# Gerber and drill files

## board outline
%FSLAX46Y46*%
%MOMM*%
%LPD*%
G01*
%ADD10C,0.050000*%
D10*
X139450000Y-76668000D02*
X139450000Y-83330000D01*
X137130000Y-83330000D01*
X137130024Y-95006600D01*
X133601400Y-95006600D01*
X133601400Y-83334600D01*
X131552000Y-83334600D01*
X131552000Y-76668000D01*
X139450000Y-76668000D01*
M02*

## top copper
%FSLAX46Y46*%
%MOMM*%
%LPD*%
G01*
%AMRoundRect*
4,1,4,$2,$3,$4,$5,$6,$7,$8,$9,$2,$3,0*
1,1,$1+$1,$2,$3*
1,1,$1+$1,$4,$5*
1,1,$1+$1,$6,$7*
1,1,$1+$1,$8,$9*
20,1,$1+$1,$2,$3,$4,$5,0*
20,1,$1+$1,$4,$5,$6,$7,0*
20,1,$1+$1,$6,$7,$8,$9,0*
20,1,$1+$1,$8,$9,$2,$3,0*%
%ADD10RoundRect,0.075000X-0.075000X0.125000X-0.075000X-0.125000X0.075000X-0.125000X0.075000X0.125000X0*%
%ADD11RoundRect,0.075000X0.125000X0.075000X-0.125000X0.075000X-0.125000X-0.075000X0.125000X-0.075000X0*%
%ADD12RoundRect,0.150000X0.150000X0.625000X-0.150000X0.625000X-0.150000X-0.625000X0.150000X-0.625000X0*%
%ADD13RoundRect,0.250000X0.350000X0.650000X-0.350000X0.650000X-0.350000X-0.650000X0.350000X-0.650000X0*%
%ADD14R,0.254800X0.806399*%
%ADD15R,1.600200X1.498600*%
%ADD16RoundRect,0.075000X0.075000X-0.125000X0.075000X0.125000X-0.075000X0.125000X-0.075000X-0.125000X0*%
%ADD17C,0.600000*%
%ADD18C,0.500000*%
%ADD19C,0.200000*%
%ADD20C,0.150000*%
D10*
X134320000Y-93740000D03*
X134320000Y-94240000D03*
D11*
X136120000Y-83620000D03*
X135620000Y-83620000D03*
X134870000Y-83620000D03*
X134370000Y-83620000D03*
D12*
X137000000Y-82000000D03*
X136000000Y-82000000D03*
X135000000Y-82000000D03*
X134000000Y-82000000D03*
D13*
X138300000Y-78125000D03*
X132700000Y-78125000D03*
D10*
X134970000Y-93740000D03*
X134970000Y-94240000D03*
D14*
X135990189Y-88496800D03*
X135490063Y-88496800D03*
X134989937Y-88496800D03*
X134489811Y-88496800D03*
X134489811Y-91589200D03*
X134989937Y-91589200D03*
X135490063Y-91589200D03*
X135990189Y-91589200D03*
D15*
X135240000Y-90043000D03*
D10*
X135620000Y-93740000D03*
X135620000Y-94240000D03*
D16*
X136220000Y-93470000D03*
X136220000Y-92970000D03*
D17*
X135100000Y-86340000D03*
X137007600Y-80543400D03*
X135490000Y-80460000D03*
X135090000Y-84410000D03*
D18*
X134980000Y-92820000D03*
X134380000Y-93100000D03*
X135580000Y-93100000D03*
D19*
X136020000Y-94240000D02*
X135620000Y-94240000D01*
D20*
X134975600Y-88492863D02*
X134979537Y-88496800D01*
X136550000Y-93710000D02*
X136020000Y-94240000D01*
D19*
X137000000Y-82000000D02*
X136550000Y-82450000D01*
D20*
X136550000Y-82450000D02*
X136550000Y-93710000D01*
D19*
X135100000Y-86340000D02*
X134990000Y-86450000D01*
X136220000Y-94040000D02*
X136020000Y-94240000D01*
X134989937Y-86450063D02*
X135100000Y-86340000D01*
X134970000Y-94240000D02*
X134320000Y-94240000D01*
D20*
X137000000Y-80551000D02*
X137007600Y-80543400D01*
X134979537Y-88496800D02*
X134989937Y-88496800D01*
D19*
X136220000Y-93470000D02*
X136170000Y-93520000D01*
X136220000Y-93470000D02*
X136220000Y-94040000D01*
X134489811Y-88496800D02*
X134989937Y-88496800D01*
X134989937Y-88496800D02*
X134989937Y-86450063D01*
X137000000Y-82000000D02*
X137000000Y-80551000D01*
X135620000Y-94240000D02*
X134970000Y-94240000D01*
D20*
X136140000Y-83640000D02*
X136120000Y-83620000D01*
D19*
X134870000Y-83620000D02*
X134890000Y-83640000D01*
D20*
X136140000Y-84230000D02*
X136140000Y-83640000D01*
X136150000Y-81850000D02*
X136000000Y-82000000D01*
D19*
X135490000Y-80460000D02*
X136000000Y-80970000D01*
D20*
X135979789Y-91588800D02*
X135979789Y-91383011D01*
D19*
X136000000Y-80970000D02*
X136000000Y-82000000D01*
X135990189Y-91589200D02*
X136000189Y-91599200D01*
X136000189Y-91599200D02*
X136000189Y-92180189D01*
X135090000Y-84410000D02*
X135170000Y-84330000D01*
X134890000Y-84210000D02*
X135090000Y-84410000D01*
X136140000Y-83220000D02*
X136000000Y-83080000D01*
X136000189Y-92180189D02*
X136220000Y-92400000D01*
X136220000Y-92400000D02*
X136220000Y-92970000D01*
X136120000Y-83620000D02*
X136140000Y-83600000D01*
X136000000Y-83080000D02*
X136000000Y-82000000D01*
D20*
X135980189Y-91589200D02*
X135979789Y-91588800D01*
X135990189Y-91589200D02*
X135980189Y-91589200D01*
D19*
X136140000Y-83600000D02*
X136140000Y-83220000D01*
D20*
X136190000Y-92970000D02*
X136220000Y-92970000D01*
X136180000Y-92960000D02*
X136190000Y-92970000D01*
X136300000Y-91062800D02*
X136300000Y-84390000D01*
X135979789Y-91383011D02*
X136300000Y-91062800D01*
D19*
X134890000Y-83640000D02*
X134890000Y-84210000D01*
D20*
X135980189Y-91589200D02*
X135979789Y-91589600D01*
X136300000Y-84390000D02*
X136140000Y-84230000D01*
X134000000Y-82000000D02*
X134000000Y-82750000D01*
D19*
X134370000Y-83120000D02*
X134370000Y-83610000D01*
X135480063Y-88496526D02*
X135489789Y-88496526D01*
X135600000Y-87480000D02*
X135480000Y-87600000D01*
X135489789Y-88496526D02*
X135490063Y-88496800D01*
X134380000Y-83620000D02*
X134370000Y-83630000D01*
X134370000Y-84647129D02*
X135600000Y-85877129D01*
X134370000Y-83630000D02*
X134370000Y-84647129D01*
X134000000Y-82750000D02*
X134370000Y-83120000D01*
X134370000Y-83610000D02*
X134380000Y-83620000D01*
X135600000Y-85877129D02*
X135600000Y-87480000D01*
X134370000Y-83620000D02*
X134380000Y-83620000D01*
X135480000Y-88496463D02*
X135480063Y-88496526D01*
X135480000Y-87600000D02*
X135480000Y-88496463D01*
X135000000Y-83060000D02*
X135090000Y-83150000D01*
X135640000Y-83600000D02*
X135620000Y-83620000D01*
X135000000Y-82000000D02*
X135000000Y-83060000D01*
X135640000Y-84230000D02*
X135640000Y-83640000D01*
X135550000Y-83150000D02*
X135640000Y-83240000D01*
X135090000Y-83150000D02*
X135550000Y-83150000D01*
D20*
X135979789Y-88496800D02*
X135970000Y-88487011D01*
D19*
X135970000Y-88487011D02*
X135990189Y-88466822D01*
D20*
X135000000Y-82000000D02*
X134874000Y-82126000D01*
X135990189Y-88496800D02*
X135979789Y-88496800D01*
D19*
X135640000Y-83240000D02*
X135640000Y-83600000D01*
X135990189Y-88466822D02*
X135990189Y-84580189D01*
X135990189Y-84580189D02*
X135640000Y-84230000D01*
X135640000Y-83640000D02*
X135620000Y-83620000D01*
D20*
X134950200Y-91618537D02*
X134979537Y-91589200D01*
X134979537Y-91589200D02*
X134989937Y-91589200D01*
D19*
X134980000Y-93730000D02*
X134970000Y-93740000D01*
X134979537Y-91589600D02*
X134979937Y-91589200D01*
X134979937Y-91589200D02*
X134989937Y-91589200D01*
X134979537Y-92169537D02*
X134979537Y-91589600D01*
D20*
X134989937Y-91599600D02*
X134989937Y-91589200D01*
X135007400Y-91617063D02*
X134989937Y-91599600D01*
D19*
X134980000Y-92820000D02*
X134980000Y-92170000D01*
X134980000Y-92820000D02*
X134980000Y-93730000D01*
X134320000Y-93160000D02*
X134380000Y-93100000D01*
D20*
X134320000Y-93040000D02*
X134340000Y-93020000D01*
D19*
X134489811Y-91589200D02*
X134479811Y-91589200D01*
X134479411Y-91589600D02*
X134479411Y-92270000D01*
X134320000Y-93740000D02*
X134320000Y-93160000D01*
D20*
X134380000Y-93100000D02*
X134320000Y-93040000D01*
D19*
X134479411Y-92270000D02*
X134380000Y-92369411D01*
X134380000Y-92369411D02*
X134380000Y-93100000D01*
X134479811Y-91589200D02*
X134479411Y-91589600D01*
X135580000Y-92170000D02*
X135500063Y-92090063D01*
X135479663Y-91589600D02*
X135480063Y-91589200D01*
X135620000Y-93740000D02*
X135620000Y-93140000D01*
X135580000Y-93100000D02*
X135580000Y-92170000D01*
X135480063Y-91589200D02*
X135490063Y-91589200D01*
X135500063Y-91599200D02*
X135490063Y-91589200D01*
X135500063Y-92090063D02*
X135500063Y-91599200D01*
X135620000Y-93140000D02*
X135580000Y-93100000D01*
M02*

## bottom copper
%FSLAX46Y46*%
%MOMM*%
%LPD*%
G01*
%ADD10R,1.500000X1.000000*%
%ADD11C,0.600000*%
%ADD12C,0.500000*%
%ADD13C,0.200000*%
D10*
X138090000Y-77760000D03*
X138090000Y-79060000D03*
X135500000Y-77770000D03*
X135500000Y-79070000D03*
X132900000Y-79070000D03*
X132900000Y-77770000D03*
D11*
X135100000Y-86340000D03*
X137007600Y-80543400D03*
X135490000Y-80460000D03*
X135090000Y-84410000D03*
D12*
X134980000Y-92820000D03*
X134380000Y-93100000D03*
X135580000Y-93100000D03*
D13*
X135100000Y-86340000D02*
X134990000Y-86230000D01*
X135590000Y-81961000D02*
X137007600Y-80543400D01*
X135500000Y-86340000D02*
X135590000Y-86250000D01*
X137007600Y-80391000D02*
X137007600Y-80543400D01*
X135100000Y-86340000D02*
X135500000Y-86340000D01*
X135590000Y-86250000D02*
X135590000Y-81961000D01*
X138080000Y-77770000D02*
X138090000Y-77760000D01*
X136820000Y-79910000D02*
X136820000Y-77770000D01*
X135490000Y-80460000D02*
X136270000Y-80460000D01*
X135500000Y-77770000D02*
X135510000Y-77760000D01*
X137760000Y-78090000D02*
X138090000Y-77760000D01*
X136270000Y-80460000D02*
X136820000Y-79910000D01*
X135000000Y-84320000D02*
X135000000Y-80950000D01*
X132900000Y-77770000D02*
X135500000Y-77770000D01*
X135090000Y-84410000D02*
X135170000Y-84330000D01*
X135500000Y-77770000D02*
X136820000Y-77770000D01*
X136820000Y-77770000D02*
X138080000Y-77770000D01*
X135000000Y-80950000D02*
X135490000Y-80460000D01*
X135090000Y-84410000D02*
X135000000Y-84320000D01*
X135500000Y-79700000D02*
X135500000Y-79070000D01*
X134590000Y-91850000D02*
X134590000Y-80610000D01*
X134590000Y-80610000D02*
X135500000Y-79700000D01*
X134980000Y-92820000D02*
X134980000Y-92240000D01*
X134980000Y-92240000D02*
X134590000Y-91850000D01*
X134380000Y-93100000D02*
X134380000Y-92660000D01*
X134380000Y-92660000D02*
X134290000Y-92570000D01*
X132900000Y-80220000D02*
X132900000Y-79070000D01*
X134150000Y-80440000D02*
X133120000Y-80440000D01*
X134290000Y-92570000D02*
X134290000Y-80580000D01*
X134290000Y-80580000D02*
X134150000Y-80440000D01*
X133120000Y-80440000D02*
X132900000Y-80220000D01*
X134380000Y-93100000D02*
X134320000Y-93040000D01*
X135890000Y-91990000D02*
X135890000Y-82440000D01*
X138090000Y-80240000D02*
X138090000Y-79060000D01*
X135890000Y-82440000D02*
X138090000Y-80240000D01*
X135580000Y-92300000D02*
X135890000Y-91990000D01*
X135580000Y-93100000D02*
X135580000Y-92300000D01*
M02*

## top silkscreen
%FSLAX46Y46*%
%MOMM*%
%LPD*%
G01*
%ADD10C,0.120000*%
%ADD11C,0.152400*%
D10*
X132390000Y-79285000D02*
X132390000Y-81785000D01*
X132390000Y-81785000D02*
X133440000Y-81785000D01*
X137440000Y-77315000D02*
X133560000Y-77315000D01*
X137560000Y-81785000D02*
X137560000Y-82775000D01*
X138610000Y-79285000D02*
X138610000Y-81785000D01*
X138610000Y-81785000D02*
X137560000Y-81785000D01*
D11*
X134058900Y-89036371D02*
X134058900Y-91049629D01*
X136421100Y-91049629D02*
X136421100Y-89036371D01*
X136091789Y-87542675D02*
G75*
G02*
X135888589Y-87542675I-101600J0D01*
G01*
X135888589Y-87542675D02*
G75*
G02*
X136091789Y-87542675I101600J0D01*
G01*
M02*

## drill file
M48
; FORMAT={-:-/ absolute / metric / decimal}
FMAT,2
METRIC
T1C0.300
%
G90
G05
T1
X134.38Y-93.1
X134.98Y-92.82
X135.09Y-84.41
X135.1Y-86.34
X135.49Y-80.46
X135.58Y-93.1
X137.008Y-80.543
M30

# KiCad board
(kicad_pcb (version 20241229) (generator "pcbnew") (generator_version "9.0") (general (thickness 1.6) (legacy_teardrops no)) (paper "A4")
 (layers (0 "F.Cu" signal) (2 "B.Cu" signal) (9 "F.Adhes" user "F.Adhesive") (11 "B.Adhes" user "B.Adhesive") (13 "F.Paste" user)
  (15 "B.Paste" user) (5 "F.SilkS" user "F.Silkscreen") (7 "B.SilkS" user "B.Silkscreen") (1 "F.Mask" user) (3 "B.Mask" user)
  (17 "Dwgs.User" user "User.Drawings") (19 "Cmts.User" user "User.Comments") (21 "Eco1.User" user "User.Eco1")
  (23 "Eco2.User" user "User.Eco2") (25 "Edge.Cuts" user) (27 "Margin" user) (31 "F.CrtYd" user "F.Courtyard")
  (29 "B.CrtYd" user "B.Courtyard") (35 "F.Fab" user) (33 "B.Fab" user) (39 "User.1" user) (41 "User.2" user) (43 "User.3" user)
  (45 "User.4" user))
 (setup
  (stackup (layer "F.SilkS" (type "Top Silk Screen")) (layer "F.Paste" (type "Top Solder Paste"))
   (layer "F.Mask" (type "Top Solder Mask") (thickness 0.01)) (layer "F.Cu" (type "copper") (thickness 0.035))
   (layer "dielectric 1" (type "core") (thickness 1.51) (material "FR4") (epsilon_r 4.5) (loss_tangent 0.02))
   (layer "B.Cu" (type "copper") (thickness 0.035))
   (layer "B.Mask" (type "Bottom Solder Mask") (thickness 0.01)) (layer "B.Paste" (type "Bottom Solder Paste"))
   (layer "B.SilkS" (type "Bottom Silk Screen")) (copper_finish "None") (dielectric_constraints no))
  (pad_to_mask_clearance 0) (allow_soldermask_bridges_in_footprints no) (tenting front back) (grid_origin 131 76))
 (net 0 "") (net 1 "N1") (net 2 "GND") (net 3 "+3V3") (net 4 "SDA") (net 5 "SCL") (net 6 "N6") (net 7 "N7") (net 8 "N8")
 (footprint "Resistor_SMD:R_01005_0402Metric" (layer "F.Cu") (at 134.32 93.99 -90)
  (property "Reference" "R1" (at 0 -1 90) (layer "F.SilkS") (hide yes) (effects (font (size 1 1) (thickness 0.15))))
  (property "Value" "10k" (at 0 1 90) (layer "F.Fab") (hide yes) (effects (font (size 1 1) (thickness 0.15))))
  (pad "" smd roundrect (at -0.275 0 270) (size 0.27 0.27) (layers "F.Paste") (roundrect_rratio 0.25))
  (pad "" smd roundrect (at 0.275 0 270) (size 0.27 0.27) (layers "F.Paste") (roundrect_rratio 0.25))
  (pad "1" smd roundrect (at -0.25 0 270) (size 0.4 0.3) (layers "F.Cu" "F.Mask") (roundrect_rratio 0.25) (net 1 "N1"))
  (pad "2" smd roundrect (at 0.25 0 270) (size 0.4 0.3) (layers "F.Cu" "F.Mask") (roundrect_rratio 0.25) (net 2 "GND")))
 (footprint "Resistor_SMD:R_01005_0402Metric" (layer "F.Cu") (at 135.87 83.62 180)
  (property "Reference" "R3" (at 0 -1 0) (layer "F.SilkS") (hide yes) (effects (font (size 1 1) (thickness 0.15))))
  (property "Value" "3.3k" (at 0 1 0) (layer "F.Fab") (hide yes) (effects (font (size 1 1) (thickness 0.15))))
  (pad "" smd roundrect (at -0.275 0 180) (size 0.27 0.27) (layers "F.Paste") (roundrect_rratio 0.25))
  (pad "" smd roundrect (at 0.275 0 180) (size 0.27 0.27) (layers "F.Paste") (roundrect_rratio 0.25))
  (pad "1" smd roundrect (at -0.25 0 180) (size 0.4 0.3) (layers "F.Cu" "F.Mask") (roundrect_rratio 0.25) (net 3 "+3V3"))
  (pad "2" smd roundrect (at 0.25 0 180) (size 0.4 0.3) (layers "F.Cu" "F.Mask") (roundrect_rratio 0.25) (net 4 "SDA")))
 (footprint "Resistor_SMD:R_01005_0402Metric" (layer "F.Cu") (at 134.62 83.62 180)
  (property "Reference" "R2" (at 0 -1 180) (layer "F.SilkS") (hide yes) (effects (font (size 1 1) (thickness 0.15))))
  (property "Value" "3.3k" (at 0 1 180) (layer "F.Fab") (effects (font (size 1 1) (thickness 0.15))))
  (pad "" smd roundrect (at -0.275 0 180) (size 0.27 0.27) (layers "F.Paste") (roundrect_rratio 0.25))
  (pad "" smd roundrect (at 0.275 0 180) (size 0.27 0.27) (layers "F.Paste") (roundrect_rratio 0.25))
  (pad "1" smd roundrect (at -0.25 0 180) (size 0.4 0.3) (layers "F.Cu" "F.Mask") (roundrect_rratio 0.25) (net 3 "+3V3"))
  (pad "2" smd roundrect (at 0.25 0 180) (size 0.4 0.3) (layers "F.Cu" "F.Mask") (roundrect_rratio 0.25) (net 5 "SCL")))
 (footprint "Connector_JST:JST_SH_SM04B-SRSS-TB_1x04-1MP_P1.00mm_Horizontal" (layer "F.Cu") (at 135.5 80 180)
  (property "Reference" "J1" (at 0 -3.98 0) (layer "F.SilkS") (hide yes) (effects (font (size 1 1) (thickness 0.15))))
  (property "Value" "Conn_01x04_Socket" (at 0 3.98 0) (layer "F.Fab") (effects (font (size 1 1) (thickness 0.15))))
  (fp_line (start 3.11 0.715) (end 3.11 -1.785) (stroke (width 0.12) (type solid)) (layer "F.SilkS"))
  (fp_line (start 3.11 -1.785) (end 2.06 -1.785) (stroke (width 0.12) (type solid)) (layer "F.SilkS"))
  (fp_line (start -1.94 2.685) (end 1.94 2.685) (stroke (width 0.12) (type solid)) (layer "F.SilkS"))
  (fp_line (start -2.06 -1.785) (end -2.06 -2.775) (stroke (width 0.12) (type solid)) (layer "F.SilkS"))
  (fp_line (start -3.11 0.715) (end -3.11 -1.785) (stroke (width 0.12) (type solid)) (layer "F.SilkS"))
  (fp_line (start -3.11 -1.785) (end -2.06 -1.785) (stroke (width 0.12) (type solid)) (layer "F.SilkS"))
  (pad "1" smd roundrect (at -1.5 -2 180) (size 0.6 1.55) (layers "F.Cu" "F.Mask" "F.Paste") (roundrect_rratio 0.25) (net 2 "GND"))
  (pad "2" smd roundrect (at -0.5 -2 180) (size 0.6 1.55) (layers "F.Cu" "F.Mask" "F.Paste") (roundrect_rratio 0.25) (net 3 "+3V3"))
  (pad "3" smd roundrect (at 0.5 -2 180) (size 0.6 1.55) (layers "F.Cu" "F.Mask" "F.Paste") (roundrect_rratio 0.25) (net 4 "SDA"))
  (pad "4" smd roundrect (at 1.5 -2 180) (size 0.6 1.55) (layers "F.Cu" "F.Mask" "F.Paste") (roundrect_rratio 0.25) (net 5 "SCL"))
  (pad "MP" smd roundrect (at -2.8 1.875 180) (size 1.2 1.8) (layers "F.Cu" "F.Mask" "F.Paste") (roundrect_rratio 0.208333))
  (pad "MP" smd roundrect (at 2.8 1.875 180) (size 1.2 1.8) (layers "F.Cu" "F.Mask" "F.Paste") (roundrect_rratio 0.208333)))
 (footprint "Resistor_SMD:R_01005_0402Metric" (layer "F.Cu") (at 134.97 93.99 -90)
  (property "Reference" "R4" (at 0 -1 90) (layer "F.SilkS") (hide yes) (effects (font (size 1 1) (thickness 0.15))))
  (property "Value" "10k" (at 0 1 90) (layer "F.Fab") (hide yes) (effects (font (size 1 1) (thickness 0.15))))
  (pad "" smd roundrect (at -0.275 0 270) (size 0.27 0.27) (layers "F.Paste") (roundrect_rratio 0.25))
  (pad "" smd roundrect (at 0.275 0 270) (size 0.27 0.27) (layers "F.Paste") (roundrect_rratio 0.25))
  (pad "1" smd roundrect (at -0.25 0 270) (size 0.4 0.3) (layers "F.Cu" "F.Mask") (roundrect_rratio 0.25) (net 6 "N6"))
  (pad "2" smd roundrect (at 0.25 0 270) (size 0.4 0.3) (layers "F.Cu" "F.Mask") (roundrect_rratio 0.25) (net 2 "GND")))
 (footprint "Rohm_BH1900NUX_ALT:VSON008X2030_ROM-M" (layer "F.Cu") (at 135.24 90.043 -90)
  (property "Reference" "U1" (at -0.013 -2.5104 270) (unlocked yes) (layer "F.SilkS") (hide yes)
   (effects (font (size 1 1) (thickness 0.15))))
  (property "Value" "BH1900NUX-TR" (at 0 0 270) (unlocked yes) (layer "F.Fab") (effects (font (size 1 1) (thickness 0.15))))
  (fp_line (start -1.006629 1.1811) (end 1.006629 1.1811) (stroke (width 0.1524) (type solid)) (layer "F.SilkS"))
  (fp_line (start 1.006629 -1.1811) (end -1.006629 -1.1811) (stroke (width 0.1524) (type solid)) (layer "F.SilkS"))
  (fp_circle (center -2.500325 -0.750189) (end -2.398725 -0.750189) (stroke (width 0.1524) (type solid)) (fill no) (layer "F.SilkS"))
  (pad "1" smd rect (at -1.5462 -0.750189 270) (size 0.806399 0.2548) (layers "F.Cu" "F.Mask" "F.Paste") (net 4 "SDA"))
  (pad "2" smd rect (at -1.5462 -0.250063 270) (size 0.806399 0.2548) (layers "F.Cu" "F.Mask" "F.Paste") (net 5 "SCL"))
  (pad "3" smd rect (at -1.5462 0.250063 270) (size 0.806399 0.2548) (layers "F.Cu" "F.Mask" "F.Paste") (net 2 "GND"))
  (pad "4" smd rect (at -1.5462 0.750189 270) (size 0.806399 0.2548) (layers "F.Cu" "F.Mask" "F.Paste") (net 2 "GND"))
  (pad "5" smd rect (at 1.5462 0.750189 270) (size 0.806399 0.2548) (layers "F.Cu" "F.Mask" "F.Paste") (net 1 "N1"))
  (pad "6" smd rect (at 1.5462 0.250063 270) (size 0.806399 0.2548) (layers "F.Cu" "F.Mask" "F.Paste") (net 6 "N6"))
  (pad "7" smd rect (at 1.5462 -0.250063 270) (size 0.806399 0.2548) (layers "F.Cu" "F.Mask" "F.Paste") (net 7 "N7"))
  (pad "8" smd rect (at 1.5462 -0.750189 270) (size 0.806399 0.2548) (layers "F.Cu" "F.Mask" "F.Paste") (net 3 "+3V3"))
  (pad "9" smd rect (at 0 0 270) (size 1.4986 1.6002) (layers "F.Cu" "F.Mask" "F.Paste") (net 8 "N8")))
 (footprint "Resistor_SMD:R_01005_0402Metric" (layer "F.Cu") (at 135.62 93.99 -90)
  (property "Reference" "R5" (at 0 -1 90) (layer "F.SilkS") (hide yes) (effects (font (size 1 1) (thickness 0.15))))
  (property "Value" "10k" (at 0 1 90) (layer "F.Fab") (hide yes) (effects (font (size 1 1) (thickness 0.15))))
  (pad "" smd roundrect (at -0.275 0 270) (size 0.27 0.27) (layers "F.Paste") (roundrect_rratio 0.25))
  (pad "" smd roundrect (at 0.275 0 270) (size 0.27 0.27) (layers "F.Paste") (roundrect_rratio 0.25))
  (pad "1" smd roundrect (at -0.25 0 270) (size 0.4 0.3) (layers "F.Cu" "F.Mask") (roundrect_rratio 0.25) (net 7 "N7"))
  (pad "2" smd roundrect (at 0.25 0 270) (size 0.4 0.3) (layers "F.Cu" "F.Mask") (roundrect_rratio 0.25) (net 2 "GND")))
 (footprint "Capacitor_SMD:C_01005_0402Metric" (layer "F.Cu") (at 136.22 93.22 90)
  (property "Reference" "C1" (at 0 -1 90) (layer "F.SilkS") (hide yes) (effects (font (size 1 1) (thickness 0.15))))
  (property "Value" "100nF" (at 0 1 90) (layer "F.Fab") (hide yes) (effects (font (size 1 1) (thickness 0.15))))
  (pad "" smd roundrect (at -0.275 0 90) (size 0.27 0.27) (layers "F.Paste") (roundrect_rratio 0.25))
  (pad "" smd roundrect (at 0.275 0 90) (size 0.27 0.27) (layers "F.Paste") (roundrect_rratio 0.25))
  (pad "1" smd roundrect (at -0.25 0 90) (size 0.4 0.3) (layers "F.Cu" "F.Mask") (roundrect_rratio 0.25) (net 2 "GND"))
  (pad "2" smd roundrect (at 0.25 0 90) (size 0.4 0.3) (layers "F.Cu" "F.Mask") (roundrect_rratio 0.25) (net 3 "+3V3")))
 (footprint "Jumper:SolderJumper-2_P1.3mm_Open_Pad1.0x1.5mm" (layer "B.Cu") (at 138.09 78.41 -90)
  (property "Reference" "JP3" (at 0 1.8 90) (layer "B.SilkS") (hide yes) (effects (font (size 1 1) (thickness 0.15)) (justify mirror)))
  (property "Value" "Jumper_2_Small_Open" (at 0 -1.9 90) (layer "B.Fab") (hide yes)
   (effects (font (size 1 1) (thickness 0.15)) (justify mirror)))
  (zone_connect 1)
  (pad "1" smd rect (at -0.65 0 270) (size 1 1.5) (layers "B.Cu" "B.Mask") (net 3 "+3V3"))
  (pad "2" smd rect (at 0.65 0 270) (size 1 1.5) (layers "B.Cu" "B.Mask") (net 7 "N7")))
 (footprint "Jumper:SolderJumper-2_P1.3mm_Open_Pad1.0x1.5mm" (layer "B.Cu") (at 135.5 78.42 -90)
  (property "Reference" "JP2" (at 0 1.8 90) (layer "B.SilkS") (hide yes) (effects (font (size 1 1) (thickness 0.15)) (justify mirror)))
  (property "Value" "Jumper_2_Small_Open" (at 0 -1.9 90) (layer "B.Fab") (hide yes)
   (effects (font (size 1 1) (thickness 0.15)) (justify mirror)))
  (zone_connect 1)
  (pad "1" smd rect (at -0.65 0 270) (size 1 1.5) (layers "B.Cu" "B.Mask") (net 3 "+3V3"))
  (pad "2" smd rect (at 0.65 0 270) (size 1 1.5) (layers "B.Cu" "B.Mask") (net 6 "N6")))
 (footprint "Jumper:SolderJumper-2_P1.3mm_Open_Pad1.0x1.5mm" (layer "B.Cu") (at 132.9 78.42 90)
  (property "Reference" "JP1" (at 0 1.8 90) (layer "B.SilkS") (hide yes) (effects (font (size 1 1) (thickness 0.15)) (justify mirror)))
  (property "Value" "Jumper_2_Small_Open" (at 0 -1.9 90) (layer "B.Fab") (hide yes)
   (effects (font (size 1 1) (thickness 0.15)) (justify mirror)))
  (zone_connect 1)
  (pad "1" smd rect (at -0.65 0 90) (size 1 1.5) (layers "B.Cu" "B.Mask") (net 1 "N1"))
  (pad "2" smd rect (at 0.65 0 90) (size 1 1.5) (layers "B.Cu" "B.Mask") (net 3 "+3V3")))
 (gr_poly
  (pts (xy 139.45 76.668) (xy 139.45 83.33) (xy 137.13 83.33) (xy 137.130024 95.0066) (xy 133.6014 95.0066) (xy 133.6014 83.3346)
   (xy 131.552 83.3346) (xy 131.552 76.668))
  (stroke (width 0.05) (type solid)) (fill no) (layer "Edge.Cuts"))
 (segment (start 136.02 94.24) (end 135.62 94.24) (width 0.2) (layer "F.Cu") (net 2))
 (segment (start 134.9756 88.492863) (end 134.979537 88.4968) (width 0.15) (layer "F.Cu") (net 2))
 (segment (start 136.55 93.71) (end 136.02 94.24) (width 0.15) (layer "F.Cu") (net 2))
 (segment (start 137 82) (end 136.55 82.45) (width 0.2) (layer "F.Cu") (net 2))
 (segment (start 136.55 82.45) (end 136.55 93.71) (width 0.15) (layer "F.Cu") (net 2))
 (segment (start 135.1 86.34) (end 134.99 86.45) (width 0.2) (layer "F.Cu") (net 2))
 (segment (start 136.22 94.04) (end 136.02 94.24) (width 0.2) (layer "F.Cu") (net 2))
 (segment (start 134.989937 86.450063) (end 135.1 86.34) (width 0.2) (layer "F.Cu") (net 2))
 (segment (start 134.97 94.24) (end 134.32 94.24) (width 0.2) (layer "F.Cu") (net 2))
 (segment (start 137 80.551) (end 137.0076 80.5434) (width 0.15) (layer "F.Cu") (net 2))
 (segment (start 134.979537 88.4968) (end 134.989937 88.4968) (width 0.15) (layer "F.Cu") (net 2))
 (segment (start 136.22 93.47) (end 136.17 93.52) (width 0.2) (layer "F.Cu") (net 2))
 (segment (start 136.22 93.47) (end 136.22 94.04) (width 0.2) (layer "F.Cu") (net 2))
 (segment (start 134.489811 88.4968) (end 134.989937 88.4968) (width 0.2) (layer "F.Cu") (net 2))
 (segment (start 134.989937 88.4968) (end 134.989937 86.450063) (width 0.2) (layer "F.Cu") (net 2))
 (segment (start 137 82) (end 137 80.551) (width 0.2) (layer "F.Cu") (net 2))
 (segment (start 135.62 94.24) (end 134.97 94.24) (width 0.2) (layer "F.Cu") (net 2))
 (via (at 135.1 86.34) (size 0.6) (drill 0.3) (layers "F.Cu" "B.Cu") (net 2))
 (via (at 137.0076 80.5434) (size 0.6) (drill 0.3) (layers "F.Cu" "B.Cu") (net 2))
 (segment (start 135.1 86.34) (end 134.99 86.23) (width 0.2) (layer "B.Cu") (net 2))
 (segment (start 135.59 81.961) (end 137.0076 80.5434) (width 0.2) (layer "B.Cu") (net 2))
 (segment (start 135.5 86.34) (end 135.59 86.25) (width 0.2) (layer "B.Cu") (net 2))
 (segment (start 137.0076 80.391) (end 137.0076 80.5434) (width 0.2) (layer "B.Cu") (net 2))
 (segment (start 135.1 86.34) (end 135.5 86.34) (width 0.2) (layer "B.Cu") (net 2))
 (segment (start 135.59 86.25) (end 135.59 81.961) (width 0.2) (layer "B.Cu") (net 2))
 (segment (start 136.14 83.64) (end 136.12 83.62) (width 0.15) (layer "F.Cu") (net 3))
 (segment (start 134.87 83.62) (end 134.89 83.64) (width 0.2) (layer "F.Cu") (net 3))
 (segment (start 136.14 84.23) (end 136.14 83.64) (width 0.15) (layer "F.Cu") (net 3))
 (segment (start 136.15 81.85) (end 136 82) (width 0.15) (layer "F.Cu") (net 3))
 (segment (start 135.49 80.46) (end 136 80.97) (width 0.2) (layer "F.Cu") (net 3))
 (segment (start 135.979789 91.5888) (end 135.979789 91.383011) (width 0.15) (layer "F.Cu") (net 3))
 (segment (start 136 80.97) (end 136 82) (width 0.2) (layer "F.Cu") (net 3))
 (segment (start 135.990189 91.5892) (end 136.000189 91.5992) (width 0.2) (layer "F.Cu") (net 3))
 (segment (start 136.000189 91.5992) (end 136.000189 92.180189) (width 0.2) (layer "F.Cu") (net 3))
 (segment (start 135.09 84.41) (end 135.17 84.33) (width 0.2) (layer "F.Cu") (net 3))
 (segment (start 134.89 84.21) (end 135.09 84.41) (width 0.2) (layer "F.Cu") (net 3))
 (segment (start 136.14 83.22) (end 136 83.08) (width 0.2) (layer "F.Cu") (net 3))
 (segment (start 136.000189 92.180189) (end 136.22 92.4) (width 0.2) (layer "F.Cu") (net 3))
 (segment (start 136.22 92.4) (end 136.22 92.97) (width 0.2) (layer "F.Cu") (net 3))
 (segment (start 136.12 83.62) (end 136.14 83.6) (width 0.2) (layer "F.Cu") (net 3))
 (segment (start 136 83.08) (end 136 82) (width 0.2) (layer "F.Cu") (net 3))
 (segment (start 135.980189 91.5892) (end 135.979789 91.5888) (width 0.15) (layer "F.Cu") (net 3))
 (segment (start 135.990189 91.5892) (end 135.980189 91.5892) (width 0.15) (layer "F.Cu") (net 3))
 (segment (start 136.14 83.6) (end 136.14 83.22) (width 0.2) (layer "F.Cu") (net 3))
 (segment (start 136.19 92.97) (end 136.22 92.97) (width 0.15) (layer "F.Cu") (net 3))
 (segment (start 136.18 92.96) (end 136.19 92.97) (width 0.15) (layer "F.Cu") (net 3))
 (segment (start 136.3 91.0628) (end 136.3 84.39) (width 0.15) (layer "F.Cu") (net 3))
 (segment (start 135.979789 91.383011) (end 136.3 91.0628) (width 0.15) (layer "F.Cu") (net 3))
 (segment (start 134.89 83.64) (end 134.89 84.21) (width 0.2) (layer "F.Cu") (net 3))
 (segment (start 135.980189 91.5892) (end 135.979789 91.5896) (width 0.15) (layer "F.Cu") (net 3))
 (segment (start 136.3 84.39) (end 136.14 84.23) (width 0.15) (layer "F.Cu") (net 3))
 (via (at 135.49 80.46) (size 0.6) (drill 0.3) (layers "F.Cu" "B.Cu") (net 3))
 (via (at 135.09 84.41) (size 0.6) (drill 0.3) (layers "F.Cu" "B.Cu") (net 3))
 (segment (start 138.08 77.77) (end 138.09 77.76) (width 0.2) (layer "B.Cu") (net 3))
 (segment (start 136.82 79.91) (end 136.82 77.77) (width 0.2) (layer "B.Cu") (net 3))
 (segment (start 135.49 80.46) (end 136.27 80.46) (width 0.2) (layer "B.Cu") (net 3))
 (segment (start 135.5 77.77) (end 135.51 77.76) (width 0.2) (layer "B.Cu") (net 3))
 (segment (start 137.76 78.09) (end 138.09 77.76) (width 0.2) (layer "B.Cu") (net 3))
 (segment (start 136.27 80.46) (end 136.82 79.91) (width 0.2) (layer "B.Cu") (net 3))
 (segment (start 135 84.32) (end 135 80.95) (width 0.2) (layer "B.Cu") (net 3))
 (segment (start 132.9 77.77) (end 135.5 77.77) (width 0.2) (layer "B.Cu") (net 3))
 (segment (start 135.09 84.41) (end 135.17 84.33) (width 0.2) (layer "B.Cu") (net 3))
 (segment (start 135.5 77.77) (end 136.82 77.77) (width 0.2) (layer "B.Cu") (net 3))
 (segment (start 136.82 77.77) (end 138.08 77.77) (width 0.2) (layer "B.Cu") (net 3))
 (segment (start 135 80.95) (end 135.49 80.46) (width 0.2) (layer "B.Cu") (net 3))
 (segment (start 135.09 84.41) (end 135 84.32) (width 0.2) (layer "B.Cu") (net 3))
 (segment (start 134 82) (end 134 82.75) (width 0.15) (layer "F.Cu") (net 5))
 (segment (start 134.37 83.12) (end 134.37 83.61) (width 0.2) (layer "F.Cu") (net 5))
 (segment (start 135.480063 88.496526) (end 135.489789 88.496526) (width 0.2) (layer "F.Cu") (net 5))
 (segment (start 135.6 87.48) (end 135.48 87.6) (width 0.2) (layer "F.Cu") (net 5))
 (segment (start 135.489789 88.496526) (end 135.490063 88.4968) (width 0.2) (layer "F.Cu") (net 5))
 (segment (start 134.38 83.62) (end 134.37 83.63) (width 0.2) (layer "F.Cu") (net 5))
 (segment (start 134.37 84.647129) (end 135.6 85.877129) (width 0.2) (layer "F.Cu") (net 5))
 (segment (start 134.37 83.63) (end 134.37 84.647129) (width 0.2) (layer "F.Cu") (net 5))
 (segment (start 134 82.75) (end 134.37 83.12) (width 0.2) (layer "F.Cu") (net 5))
 (segment (start 134.37 83.61) (end 134.38 83.62) (width 0.2) (layer "F.Cu") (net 5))
 (segment (start 135.6 85.877129) (end 135.6 87.48) (width 0.2) (layer "F.Cu") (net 5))
 (segment (start 134.37 83.62) (end 134.38 83.62) (width 0.2) (layer "F.Cu") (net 5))
 (segment (start 135.48 88.496463) (end 135.480063 88.496526) (width 0.2) (layer "F.Cu") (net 5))
 (segment (start 135.48 87.6) (end 135.48 88.496463) (width 0.2) (layer "F.Cu") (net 5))
 (segment (start 135 83.06) (end 135.09 83.15) (width 0.2) (layer "F.Cu") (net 4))
 (segment (start 135.64 83.6) (end 135.62 83.62) (width 0.2) (layer "F.Cu") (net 4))
 (segment (start 135 82) (end 135 83.06) (width 0.2) (layer "F.Cu") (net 4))
 (segment (start 135.64 84.23) (end 135.64 83.64) (width 0.2) (layer "F.Cu") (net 4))
 (segment (start 135.55 83.15) (end 135.64 83.24) (width 0.2) (layer "F.Cu") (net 4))
 (segment (start 135.09 83.15) (end 135.55 83.15) (width 0.2) (layer "F.Cu") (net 4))
 (segment (start 135.979789 88.4968) (end 135.97 88.487011) (width 0.15) (layer "F.Cu") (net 4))
 (segment (start 135.97 88.487011) (end 135.990189 88.466822) (width 0.2) (layer "F.Cu") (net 4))
 (segment (start 135 82) (end 134.874 82.126) (width 0.15) (layer "F.Cu") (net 4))
 (segment (start 135.990189 88.4968) (end 135.979789 88.4968) (width 0.15) (layer "F.Cu") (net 4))
 (segment (start 135.64 83.24) (end 135.64 83.6) (width 0.2) (layer "F.Cu") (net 4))
 (segment (start 135.990189 88.466822) (end 135.990189 84.580189) (width 0.2) (layer "F.Cu") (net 4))
 (segment (start 135.990189 84.580189) (end 135.64 84.23) (width 0.2) (layer "F.Cu") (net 4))
 (segment (start 135.64 83.64) (end 135.62 83.62) (width 0.2) (layer "F.Cu") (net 4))
 (segment (start 134.9502 91.618537) (end 134.979537 91.5892) (width 0.15) (layer "F.Cu") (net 6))
 (segment (start 134.979537 91.5892) (end 134.989937 91.5892) (width 0.15) (layer "F.Cu") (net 6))
 (segment (start 134.98 93.73) (end 134.97 93.74) (width 0.2) (layer "F.Cu") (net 6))
 (segment (start 134.979537 91.5896) (end 134.979937 91.5892) (width 0.2) (layer "F.Cu") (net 6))
 (segment (start 134.979937 91.5892) (end 134.989937 91.5892) (width 0.2) (layer "F.Cu") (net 6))
 (segment (start 134.979537 92.169537) (end 134.979537 91.5896) (width 0.2) (layer "F.Cu") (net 6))
 (segment (start 134.989937 91.5996) (end 134.989937 91.5892) (width 0.15) (layer "F.Cu") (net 6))
 (segment (start 135.0074 91.617063) (end 134.989937 91.5996) (width 0.15) (layer "F.Cu") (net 6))
 (segment (start 134.98 92.82) (end 134.98 92.17) (width 0.2) (layer "F.Cu") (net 6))
 (segment (start 134.98 92.82) (end 134.98 93.73) (width 0.2) (layer "F.Cu") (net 6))
 (via (at 134.98 92.82) (size 0.5) (drill 0.3) (layers "F.Cu" "B.Cu") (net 6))
 (segment (start 135.5 79.7) (end 135.5 79.07) (width 0.2) (layer "B.Cu") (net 6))
 (segment (start 134.59 91.85) (end 134.59 80.61) (width 0.2) (layer "B.Cu") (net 6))
 (segment (start 134.59 80.61) (end 135.5 79.7) (width 0.2) (layer "B.Cu") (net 6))
 (segment (start 134.98 92.82) (end 134.98 92.24) (width 0.2) (layer "B.Cu") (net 6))
 (segment (start 134.98 92.24) (end 134.59 91.85) (width 0.2) (layer "B.Cu") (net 6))
 (segment (start 134.32 93.16) (end 134.38 93.1) (width 0.2) (layer "F.Cu") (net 1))
 (segment (start 134.32 93.04) (end 134.34 93.02) (width 0.15) (layer "F.Cu") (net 1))
 (segment (start 134.489811 91.5892) (end 134.479811 91.5892) (width 0.2) (layer "F.Cu") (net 1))
 (segment (start 134.479411 91.5896) (end 134.479411 92.27) (width 0.2) (layer "F.Cu") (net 1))
 (segment (start 134.32 93.74) (end 134.32 93.16) (width 0.2) (layer "F.Cu") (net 1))
 (segment (start 134.38 93.1) (end 134.32 93.04) (width 0.15) (layer "F.Cu") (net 1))
 (segment (start 134.479411 92.27) (end 134.38 92.369411) (width 0.2) (layer "F.Cu") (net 1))
 (segment (start 134.38 92.369411) (end 134.38 93.1) (width 0.2) (layer "F.Cu") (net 1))
 (segment (start 134.479811 91.5892) (end 134.479411 91.5896) (width 0.2) (layer "F.Cu") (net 1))
 (via (at 134.38 93.1) (size 0.5) (drill 0.3) (layers "F.Cu" "B.Cu") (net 1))
 (segment (start 134.38 93.1) (end 134.38 92.66) (width 0.2) (layer "B.Cu") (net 1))
 (segment (start 134.38 92.66) (end 134.29 92.57) (width 0.2) (layer "B.Cu") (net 1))
 (segment (start 132.9 80.22) (end 132.9 79.07) (width 0.2) (layer "B.Cu") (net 1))
 (segment (start 134.15 80.44) (end 133.12 80.44) (width 0.2) (layer "B.Cu") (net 1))
 (segment (start 134.29 92.57) (end 134.29 80.58) (width 0.2) (layer "B.Cu") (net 1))
 (segment (start 134.29 80.58) (end 134.15 80.44) (width 0.2) (layer "B.Cu") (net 1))
 (segment (start 133.12 80.44) (end 132.9 80.22) (width 0.2) (layer "B.Cu") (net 1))
 (segment (start 134.38 93.1) (end 134.32 93.04) (width 0.2) (layer "B.Cu") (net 1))
 (segment (start 135.58 92.17) (end 135.500063 92.090063) (width 0.2) (layer "F.Cu") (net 7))
 (segment (start 135.479663 91.5896) (end 135.480063 91.5892) (width 0.2) (layer "F.Cu") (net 7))
 (segment (start 135.62 93.74) (end 135.62 93.14) (width 0.2) (layer "F.Cu") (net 7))
 (segment (start 135.58 93.1) (end 135.58 92.17) (width 0.2) (layer "F.Cu") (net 7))
 (segment (start 135.480063 91.5892) (end 135.490063 91.5892) (width 0.2) (layer "F.Cu") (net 7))
 (segment (start 135.500063 91.5992) (end 135.490063 91.5892) (width 0.2) (layer "F.Cu") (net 7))
 (segment (start 135.500063 92.090063) (end 135.500063 91.5992) (width 0.2) (layer "F.Cu") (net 7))
 (segment (start 135.62 93.14) (end 135.58 93.1) (width 0.2) (layer "F.Cu") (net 7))
 (via (at 135.58 93.1) (size 0.5) (drill 0.3) (layers "F.Cu" "B.Cu") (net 7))
 (segment (start 135.89 91.99) (end 135.89 82.44) (width 0.2) (layer "B.Cu") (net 7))
 (segment (start 138.09 80.24) (end 138.09 79.06) (width 0.2) (layer "B.Cu") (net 7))
 (segment (start 135.89 82.44) (end 138.09 80.24) (width 0.2) (layer "B.Cu") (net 7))
 (segment (start 135.58 92.3) (end 135.89 91.99) (width 0.2) (layer "B.Cu") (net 7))
 (segment (start 135.58 93.1) (end 135.58 92.3) (width 0.2) (layer "B.Cu") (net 7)))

